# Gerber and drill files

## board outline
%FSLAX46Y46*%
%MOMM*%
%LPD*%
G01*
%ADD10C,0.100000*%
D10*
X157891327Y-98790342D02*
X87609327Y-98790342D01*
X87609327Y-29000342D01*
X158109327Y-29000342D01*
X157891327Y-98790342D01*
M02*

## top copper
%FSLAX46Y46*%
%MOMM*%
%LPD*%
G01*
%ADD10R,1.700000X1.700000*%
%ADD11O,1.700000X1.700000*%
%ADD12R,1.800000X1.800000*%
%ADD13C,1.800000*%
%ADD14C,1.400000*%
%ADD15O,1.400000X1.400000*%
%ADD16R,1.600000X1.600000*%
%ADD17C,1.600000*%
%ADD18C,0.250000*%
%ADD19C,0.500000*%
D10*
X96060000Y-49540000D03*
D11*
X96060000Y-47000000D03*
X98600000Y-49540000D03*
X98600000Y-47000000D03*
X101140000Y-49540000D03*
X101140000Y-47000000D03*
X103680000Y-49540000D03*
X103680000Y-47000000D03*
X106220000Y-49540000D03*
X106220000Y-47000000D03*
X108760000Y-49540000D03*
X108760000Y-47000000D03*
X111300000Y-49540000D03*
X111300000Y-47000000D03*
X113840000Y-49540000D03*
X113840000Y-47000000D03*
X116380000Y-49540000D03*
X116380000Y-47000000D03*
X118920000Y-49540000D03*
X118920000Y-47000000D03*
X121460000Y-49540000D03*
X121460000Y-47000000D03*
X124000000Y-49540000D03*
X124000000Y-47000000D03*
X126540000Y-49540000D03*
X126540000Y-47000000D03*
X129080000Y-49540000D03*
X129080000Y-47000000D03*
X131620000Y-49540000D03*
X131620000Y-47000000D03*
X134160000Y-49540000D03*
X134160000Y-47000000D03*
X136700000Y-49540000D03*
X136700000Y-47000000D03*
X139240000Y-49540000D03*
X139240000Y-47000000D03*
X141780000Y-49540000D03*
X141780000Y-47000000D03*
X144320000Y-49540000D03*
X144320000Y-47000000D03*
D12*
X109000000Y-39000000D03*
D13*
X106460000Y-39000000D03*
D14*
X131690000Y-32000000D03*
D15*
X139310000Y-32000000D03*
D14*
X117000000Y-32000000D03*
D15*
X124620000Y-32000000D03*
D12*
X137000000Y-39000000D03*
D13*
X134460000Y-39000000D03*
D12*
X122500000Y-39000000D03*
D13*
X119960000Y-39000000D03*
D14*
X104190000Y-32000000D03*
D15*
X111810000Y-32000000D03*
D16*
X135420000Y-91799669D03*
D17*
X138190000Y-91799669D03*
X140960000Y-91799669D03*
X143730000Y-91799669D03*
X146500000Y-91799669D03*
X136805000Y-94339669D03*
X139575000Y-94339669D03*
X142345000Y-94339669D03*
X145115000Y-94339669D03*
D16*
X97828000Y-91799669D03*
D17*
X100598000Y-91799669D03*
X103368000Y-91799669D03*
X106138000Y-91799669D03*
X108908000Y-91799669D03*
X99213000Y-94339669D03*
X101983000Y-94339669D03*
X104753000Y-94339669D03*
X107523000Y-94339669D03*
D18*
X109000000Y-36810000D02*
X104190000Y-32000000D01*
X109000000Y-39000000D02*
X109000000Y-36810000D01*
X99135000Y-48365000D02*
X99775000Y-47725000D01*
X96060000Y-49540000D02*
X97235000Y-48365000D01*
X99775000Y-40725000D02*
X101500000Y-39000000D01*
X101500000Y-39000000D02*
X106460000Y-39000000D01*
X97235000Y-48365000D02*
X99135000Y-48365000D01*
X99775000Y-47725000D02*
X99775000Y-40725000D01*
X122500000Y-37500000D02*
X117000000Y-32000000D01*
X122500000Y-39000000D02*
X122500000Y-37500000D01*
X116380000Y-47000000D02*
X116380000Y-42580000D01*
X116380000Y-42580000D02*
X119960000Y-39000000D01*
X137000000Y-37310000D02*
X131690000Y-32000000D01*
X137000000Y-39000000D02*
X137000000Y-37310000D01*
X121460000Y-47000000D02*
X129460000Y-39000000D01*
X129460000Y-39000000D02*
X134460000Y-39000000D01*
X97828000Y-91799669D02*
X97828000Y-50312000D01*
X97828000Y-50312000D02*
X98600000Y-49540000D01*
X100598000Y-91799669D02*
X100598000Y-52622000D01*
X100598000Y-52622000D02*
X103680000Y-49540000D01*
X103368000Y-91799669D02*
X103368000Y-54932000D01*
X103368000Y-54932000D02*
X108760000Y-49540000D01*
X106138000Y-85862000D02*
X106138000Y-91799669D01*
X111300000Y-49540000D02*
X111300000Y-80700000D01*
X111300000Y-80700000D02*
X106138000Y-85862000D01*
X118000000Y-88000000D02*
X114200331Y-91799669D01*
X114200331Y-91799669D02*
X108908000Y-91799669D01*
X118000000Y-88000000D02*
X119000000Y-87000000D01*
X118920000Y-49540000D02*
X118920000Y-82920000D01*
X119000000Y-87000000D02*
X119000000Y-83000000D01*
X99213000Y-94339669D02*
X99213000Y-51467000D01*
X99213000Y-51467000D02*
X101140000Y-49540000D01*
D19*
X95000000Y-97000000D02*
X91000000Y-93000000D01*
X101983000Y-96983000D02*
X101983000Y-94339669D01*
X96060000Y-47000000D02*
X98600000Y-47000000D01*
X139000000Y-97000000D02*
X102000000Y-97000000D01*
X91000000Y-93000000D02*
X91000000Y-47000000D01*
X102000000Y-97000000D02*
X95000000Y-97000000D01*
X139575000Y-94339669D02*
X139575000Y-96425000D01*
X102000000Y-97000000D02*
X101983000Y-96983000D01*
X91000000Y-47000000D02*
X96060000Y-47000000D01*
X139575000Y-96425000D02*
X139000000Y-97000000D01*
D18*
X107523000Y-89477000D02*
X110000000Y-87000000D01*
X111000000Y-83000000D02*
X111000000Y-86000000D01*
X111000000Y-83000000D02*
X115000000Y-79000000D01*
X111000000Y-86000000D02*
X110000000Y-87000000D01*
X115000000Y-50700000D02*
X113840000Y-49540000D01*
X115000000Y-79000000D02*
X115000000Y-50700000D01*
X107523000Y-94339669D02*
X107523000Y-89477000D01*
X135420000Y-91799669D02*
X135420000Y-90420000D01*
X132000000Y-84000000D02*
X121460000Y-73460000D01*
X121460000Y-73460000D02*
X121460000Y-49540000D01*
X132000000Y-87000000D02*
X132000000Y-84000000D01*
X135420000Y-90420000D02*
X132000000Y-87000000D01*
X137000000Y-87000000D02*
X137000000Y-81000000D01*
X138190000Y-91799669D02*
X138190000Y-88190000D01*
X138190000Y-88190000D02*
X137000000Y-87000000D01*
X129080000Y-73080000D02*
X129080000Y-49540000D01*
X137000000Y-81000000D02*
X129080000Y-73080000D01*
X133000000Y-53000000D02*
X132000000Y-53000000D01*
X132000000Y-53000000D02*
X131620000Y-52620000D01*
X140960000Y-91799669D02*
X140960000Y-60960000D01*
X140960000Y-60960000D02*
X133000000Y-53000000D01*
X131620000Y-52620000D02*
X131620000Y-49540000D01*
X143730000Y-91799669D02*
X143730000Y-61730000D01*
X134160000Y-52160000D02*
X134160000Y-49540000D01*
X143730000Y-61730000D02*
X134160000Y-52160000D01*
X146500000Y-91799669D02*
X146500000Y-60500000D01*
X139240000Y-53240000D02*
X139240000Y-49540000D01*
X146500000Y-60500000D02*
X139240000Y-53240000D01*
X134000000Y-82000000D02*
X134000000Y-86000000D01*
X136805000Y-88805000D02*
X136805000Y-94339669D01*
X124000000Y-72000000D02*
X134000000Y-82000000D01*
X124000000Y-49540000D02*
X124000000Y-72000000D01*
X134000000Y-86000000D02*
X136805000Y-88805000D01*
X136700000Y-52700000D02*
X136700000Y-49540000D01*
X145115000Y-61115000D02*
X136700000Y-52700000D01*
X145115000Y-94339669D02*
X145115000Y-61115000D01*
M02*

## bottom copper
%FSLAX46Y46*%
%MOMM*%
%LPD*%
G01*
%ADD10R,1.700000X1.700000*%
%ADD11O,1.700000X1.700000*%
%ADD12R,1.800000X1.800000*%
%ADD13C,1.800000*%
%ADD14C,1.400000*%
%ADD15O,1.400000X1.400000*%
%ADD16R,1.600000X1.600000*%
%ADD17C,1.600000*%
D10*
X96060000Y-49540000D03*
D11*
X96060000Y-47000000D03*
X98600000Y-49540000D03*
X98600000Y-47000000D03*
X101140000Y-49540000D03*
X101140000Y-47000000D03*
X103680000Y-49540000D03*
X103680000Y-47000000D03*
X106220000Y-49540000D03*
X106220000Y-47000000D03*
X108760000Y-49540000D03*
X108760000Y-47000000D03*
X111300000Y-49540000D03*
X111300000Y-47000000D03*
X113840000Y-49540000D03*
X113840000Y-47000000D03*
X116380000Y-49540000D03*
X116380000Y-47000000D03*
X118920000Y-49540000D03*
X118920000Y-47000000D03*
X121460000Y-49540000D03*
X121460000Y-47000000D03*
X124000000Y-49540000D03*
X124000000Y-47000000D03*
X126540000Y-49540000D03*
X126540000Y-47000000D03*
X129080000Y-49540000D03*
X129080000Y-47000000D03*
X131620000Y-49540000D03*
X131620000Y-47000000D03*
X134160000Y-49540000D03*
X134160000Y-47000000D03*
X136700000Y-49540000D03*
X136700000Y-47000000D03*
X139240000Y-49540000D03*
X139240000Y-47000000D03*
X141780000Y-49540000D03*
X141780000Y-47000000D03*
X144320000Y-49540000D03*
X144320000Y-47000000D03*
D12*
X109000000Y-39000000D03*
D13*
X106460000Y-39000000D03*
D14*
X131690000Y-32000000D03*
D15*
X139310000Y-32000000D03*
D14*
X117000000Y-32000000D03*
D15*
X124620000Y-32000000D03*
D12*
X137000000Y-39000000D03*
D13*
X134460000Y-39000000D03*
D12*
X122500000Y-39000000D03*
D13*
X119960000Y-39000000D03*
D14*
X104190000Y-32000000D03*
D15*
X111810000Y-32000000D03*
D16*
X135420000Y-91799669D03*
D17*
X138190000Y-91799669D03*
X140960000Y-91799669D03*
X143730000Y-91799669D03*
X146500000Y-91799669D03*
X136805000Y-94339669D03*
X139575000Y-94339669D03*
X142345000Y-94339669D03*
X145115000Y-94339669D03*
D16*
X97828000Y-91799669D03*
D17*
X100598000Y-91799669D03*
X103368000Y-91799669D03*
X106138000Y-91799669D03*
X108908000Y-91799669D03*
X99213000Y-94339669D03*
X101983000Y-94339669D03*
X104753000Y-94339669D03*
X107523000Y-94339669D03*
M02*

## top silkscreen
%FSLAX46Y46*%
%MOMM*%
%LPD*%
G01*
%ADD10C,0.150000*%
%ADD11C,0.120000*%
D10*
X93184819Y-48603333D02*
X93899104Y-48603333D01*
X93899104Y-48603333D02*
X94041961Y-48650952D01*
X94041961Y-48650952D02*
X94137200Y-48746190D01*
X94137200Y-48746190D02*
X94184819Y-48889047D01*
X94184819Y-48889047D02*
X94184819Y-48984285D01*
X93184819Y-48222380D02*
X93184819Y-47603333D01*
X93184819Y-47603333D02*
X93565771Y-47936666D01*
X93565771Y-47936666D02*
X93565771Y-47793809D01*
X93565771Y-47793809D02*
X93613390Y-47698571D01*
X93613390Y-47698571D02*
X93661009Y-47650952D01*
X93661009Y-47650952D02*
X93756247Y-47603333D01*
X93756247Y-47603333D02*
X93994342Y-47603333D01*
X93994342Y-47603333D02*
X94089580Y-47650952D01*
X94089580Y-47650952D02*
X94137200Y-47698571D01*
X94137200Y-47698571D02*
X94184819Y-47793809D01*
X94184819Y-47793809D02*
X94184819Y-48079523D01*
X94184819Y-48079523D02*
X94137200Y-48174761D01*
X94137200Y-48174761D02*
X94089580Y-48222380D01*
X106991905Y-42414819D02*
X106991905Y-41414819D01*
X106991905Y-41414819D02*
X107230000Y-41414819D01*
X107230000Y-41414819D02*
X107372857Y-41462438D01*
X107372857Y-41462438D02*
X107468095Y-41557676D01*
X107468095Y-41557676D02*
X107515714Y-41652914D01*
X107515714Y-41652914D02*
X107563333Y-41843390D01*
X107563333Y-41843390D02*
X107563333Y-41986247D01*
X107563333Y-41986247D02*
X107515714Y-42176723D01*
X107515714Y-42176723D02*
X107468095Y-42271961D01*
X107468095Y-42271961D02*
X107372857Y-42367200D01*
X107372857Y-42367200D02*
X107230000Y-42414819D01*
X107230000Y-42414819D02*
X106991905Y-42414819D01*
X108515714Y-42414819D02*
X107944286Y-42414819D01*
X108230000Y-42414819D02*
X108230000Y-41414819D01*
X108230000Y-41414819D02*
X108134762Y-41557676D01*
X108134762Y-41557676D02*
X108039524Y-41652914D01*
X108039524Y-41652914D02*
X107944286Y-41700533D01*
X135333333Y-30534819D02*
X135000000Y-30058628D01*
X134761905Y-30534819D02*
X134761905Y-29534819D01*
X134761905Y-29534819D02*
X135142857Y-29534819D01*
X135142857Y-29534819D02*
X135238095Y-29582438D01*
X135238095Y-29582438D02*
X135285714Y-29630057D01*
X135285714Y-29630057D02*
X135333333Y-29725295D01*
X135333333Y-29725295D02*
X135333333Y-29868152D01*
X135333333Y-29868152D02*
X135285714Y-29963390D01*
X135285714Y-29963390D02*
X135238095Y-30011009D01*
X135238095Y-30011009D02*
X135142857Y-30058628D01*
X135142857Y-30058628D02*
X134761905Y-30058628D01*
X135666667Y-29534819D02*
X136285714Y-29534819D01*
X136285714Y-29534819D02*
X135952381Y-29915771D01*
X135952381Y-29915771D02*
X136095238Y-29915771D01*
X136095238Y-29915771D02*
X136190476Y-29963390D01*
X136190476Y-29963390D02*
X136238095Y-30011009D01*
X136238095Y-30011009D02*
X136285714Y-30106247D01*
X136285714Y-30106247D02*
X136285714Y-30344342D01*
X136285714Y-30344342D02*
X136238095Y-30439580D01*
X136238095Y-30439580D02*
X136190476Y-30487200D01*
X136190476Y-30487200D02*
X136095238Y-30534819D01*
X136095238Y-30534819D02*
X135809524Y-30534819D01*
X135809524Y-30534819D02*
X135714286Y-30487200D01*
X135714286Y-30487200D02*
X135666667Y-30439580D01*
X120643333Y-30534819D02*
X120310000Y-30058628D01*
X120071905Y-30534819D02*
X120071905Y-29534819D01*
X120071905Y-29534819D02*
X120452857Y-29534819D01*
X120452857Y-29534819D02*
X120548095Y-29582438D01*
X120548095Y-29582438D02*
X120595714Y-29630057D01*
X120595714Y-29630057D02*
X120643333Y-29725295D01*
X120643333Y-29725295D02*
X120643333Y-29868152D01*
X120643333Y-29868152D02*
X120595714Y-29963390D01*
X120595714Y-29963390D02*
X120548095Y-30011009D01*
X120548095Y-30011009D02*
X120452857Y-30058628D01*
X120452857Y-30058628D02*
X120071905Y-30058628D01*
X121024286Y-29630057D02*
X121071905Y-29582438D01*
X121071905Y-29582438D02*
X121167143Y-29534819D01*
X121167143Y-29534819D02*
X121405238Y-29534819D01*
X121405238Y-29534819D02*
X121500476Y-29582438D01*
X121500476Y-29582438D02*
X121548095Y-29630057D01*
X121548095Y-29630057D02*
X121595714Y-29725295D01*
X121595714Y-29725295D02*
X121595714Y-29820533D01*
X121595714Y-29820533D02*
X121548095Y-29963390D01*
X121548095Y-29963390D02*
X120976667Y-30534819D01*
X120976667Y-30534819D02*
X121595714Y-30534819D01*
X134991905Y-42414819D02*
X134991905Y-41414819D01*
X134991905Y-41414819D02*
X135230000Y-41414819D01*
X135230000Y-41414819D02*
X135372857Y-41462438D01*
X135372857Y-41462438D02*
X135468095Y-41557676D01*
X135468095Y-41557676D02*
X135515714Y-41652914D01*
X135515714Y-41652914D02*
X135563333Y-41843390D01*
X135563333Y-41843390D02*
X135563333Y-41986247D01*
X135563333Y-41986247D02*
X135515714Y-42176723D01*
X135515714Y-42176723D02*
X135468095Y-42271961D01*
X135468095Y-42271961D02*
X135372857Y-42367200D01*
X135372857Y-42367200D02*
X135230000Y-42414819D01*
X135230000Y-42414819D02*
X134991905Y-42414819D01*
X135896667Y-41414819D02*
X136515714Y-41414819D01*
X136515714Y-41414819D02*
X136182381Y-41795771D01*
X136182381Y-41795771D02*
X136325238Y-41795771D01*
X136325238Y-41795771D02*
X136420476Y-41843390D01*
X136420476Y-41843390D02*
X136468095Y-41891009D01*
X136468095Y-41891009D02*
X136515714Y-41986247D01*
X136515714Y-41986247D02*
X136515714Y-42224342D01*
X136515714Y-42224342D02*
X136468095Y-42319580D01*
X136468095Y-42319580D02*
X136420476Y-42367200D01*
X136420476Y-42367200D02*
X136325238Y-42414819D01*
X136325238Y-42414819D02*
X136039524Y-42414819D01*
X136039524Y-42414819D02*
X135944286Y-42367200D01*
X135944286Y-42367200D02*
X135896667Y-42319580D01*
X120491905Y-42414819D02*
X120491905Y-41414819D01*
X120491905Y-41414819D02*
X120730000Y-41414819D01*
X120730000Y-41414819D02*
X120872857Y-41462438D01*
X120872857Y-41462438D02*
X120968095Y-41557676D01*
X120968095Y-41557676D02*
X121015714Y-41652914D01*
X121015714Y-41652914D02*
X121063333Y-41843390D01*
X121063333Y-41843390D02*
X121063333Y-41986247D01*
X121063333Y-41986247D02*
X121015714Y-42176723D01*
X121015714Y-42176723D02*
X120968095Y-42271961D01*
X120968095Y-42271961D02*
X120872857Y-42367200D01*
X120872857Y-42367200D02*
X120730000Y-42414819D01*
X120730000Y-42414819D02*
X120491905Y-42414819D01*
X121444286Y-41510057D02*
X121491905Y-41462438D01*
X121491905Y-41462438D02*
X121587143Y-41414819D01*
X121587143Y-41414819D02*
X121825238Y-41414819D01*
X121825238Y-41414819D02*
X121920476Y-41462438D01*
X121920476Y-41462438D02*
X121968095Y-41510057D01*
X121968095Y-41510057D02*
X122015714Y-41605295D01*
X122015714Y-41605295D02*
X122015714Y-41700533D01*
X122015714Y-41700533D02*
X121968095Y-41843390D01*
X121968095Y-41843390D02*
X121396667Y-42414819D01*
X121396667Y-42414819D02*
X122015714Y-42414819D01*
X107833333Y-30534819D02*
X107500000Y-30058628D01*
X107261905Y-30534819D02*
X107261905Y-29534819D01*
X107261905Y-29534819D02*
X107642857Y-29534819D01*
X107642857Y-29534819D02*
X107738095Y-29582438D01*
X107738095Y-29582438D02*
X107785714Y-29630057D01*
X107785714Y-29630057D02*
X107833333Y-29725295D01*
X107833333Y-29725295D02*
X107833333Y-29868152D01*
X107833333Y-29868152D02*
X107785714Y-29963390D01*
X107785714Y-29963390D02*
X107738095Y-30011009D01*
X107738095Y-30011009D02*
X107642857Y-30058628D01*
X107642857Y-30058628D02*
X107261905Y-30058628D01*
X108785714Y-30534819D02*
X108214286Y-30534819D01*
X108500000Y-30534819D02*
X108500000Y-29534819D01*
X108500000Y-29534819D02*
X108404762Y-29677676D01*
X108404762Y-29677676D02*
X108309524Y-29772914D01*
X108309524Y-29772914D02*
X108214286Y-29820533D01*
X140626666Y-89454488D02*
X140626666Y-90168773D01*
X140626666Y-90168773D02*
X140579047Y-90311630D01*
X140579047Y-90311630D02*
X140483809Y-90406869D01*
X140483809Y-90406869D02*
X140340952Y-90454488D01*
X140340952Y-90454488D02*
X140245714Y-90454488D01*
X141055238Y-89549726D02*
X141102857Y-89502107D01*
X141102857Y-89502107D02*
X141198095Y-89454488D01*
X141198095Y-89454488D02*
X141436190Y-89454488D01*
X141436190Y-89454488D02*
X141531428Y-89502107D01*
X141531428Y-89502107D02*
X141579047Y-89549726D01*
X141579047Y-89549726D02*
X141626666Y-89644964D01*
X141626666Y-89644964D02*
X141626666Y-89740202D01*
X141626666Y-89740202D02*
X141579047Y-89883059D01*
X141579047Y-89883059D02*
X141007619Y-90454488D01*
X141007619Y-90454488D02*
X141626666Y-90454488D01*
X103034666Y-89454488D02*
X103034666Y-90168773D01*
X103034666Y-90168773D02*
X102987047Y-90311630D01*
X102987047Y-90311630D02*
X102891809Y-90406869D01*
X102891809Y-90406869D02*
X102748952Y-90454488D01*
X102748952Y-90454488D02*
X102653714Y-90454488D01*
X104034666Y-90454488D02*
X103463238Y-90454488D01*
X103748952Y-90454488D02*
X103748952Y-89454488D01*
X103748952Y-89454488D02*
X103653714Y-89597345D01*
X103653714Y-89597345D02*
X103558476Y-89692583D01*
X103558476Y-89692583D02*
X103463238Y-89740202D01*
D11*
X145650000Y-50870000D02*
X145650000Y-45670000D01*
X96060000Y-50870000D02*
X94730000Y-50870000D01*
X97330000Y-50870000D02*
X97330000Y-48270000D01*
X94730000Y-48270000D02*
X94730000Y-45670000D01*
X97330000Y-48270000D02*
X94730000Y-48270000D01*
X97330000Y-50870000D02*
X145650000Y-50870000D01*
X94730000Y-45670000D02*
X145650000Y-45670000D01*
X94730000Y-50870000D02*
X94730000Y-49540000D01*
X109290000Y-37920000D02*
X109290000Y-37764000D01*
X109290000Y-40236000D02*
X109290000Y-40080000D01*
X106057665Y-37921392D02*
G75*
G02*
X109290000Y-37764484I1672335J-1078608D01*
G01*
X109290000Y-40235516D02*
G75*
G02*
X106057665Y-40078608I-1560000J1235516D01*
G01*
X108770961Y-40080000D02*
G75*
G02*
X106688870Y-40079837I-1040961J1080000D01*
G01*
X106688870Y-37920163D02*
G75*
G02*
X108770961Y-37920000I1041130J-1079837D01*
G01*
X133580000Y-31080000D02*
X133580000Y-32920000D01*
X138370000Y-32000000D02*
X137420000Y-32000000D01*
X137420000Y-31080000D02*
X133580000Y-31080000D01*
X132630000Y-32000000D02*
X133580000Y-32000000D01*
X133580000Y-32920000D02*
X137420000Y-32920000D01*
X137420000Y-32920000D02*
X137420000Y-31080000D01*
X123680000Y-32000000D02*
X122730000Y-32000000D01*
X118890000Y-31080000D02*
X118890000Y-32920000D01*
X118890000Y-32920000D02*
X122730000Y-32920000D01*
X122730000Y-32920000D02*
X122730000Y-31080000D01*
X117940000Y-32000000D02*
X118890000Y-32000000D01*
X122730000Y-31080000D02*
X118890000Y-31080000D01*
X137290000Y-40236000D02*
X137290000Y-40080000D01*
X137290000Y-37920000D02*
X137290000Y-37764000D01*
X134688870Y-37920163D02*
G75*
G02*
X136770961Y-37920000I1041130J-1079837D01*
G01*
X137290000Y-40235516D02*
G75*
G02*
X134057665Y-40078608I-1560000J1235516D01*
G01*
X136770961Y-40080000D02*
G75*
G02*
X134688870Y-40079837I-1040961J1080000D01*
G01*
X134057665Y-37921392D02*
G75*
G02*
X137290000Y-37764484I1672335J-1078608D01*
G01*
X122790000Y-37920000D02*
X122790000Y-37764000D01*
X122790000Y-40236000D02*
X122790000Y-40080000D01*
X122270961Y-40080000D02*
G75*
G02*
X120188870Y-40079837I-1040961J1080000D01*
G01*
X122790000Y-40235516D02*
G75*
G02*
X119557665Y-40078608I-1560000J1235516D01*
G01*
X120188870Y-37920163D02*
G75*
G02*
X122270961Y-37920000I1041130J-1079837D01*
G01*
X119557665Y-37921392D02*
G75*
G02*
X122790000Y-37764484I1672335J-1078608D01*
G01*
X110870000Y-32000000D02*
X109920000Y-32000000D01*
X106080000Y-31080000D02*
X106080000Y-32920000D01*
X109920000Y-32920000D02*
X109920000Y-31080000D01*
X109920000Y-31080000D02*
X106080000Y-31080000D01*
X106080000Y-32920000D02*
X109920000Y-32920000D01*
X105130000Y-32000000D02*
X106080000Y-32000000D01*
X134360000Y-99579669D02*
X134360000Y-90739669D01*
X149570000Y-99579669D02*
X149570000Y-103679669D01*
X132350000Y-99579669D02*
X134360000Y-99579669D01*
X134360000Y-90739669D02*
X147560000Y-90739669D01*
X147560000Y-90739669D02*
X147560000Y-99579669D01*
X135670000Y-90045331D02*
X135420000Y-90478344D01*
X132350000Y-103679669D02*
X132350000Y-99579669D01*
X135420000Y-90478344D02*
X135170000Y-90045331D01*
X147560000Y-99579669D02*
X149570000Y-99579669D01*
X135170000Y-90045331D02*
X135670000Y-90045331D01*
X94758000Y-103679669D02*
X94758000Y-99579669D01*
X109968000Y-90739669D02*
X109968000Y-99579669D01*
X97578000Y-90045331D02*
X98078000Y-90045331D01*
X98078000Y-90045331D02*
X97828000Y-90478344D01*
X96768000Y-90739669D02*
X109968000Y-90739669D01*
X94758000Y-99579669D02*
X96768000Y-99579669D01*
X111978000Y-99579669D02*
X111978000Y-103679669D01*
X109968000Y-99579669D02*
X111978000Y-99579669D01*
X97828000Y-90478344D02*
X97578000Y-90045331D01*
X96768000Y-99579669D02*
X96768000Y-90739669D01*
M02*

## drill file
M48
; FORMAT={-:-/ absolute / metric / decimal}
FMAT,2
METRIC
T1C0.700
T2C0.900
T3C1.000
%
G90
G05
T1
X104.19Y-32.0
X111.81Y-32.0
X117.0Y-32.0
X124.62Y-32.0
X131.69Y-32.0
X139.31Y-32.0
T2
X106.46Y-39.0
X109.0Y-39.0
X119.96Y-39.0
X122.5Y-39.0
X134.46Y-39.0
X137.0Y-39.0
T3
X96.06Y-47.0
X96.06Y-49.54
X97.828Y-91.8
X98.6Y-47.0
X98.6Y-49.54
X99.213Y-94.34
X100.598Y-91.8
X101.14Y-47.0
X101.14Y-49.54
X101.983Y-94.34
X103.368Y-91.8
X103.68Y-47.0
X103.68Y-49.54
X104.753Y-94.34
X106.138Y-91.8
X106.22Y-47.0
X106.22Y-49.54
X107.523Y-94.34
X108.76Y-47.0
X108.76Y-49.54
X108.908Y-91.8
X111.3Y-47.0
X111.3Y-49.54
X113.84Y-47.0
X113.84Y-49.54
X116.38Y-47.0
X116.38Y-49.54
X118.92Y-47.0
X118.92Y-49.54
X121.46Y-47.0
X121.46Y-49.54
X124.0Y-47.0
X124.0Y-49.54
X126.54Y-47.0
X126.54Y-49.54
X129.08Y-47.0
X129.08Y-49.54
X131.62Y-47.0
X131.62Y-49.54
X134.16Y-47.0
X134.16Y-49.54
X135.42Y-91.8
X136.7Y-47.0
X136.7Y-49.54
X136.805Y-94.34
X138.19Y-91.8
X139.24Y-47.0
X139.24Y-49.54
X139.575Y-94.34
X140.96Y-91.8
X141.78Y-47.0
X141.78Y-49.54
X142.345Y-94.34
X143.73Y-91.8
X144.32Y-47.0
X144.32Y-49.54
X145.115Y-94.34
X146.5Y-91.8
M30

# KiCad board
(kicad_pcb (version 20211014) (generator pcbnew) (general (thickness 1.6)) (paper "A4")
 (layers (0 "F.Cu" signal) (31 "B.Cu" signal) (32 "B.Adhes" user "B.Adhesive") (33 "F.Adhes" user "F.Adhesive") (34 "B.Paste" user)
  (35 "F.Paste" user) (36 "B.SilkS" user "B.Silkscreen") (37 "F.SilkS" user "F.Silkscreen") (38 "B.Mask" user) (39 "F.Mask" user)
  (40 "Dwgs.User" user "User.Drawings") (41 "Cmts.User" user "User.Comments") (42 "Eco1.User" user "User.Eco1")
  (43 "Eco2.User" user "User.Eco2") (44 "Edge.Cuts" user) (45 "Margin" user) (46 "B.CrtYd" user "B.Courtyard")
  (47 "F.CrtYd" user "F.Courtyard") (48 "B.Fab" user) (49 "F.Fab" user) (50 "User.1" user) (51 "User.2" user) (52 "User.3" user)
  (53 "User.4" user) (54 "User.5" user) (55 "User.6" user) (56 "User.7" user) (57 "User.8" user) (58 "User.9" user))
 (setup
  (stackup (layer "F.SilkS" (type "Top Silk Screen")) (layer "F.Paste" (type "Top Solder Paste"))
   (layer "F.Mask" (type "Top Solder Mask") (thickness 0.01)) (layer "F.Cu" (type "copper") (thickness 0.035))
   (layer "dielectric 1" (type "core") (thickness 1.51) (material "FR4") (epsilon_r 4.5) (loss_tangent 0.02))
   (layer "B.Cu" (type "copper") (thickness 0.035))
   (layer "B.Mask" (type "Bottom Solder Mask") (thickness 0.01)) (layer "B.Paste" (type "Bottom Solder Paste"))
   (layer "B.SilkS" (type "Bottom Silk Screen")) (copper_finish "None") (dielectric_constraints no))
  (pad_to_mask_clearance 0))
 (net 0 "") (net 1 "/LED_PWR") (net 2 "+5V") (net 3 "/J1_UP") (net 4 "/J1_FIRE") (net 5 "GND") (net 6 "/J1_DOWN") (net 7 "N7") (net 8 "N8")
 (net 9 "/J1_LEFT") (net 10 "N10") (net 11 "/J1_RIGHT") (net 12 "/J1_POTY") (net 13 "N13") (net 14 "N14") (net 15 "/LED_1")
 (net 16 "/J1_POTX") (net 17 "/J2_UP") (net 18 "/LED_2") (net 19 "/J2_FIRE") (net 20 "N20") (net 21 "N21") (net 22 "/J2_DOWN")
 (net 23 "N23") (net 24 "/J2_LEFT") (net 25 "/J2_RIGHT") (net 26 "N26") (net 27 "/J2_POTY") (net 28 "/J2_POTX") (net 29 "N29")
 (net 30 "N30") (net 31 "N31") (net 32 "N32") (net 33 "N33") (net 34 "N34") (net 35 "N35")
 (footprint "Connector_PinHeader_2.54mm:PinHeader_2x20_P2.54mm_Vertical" (layer "F.Cu") (at 96.06 49.54 90)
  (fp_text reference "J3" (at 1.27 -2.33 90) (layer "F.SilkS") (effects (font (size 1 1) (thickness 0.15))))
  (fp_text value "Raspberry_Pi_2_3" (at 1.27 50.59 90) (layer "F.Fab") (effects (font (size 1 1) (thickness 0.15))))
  (fp_line (start -1.33 49.59) (end 3.87 49.59) (layer "F.SilkS") (width 0.12))
  (fp_line (start -1.33 0) (end -1.33 -1.33) (layer "F.SilkS") (width 0.12))
  (fp_line (start -1.33 1.27) (end 1.27 1.27) (layer "F.SilkS") (width 0.12))
  (fp_line (start 1.27 -1.33) (end 3.87 -1.33) (layer "F.SilkS") (width 0.12))
  (fp_line (start 1.27 1.27) (end 1.27 -1.33) (layer "F.SilkS") (width 0.12))
  (fp_line (start -1.33 1.27) (end -1.33 49.59) (layer "F.SilkS") (width 0.12))
  (fp_line (start 3.87 -1.33) (end 3.87 49.59) (layer "F.SilkS") (width 0.12))
  (fp_line (start -1.33 -1.33) (end 0 -1.33) (layer "F.SilkS") (width 0.12))
  (pad "1" thru_hole rect (at 0 0 90) (size 1.7 1.7) (drill 1) (layers *.Cu *.Mask) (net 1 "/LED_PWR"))
  (pad "2" thru_hole oval (at 2.54 0 90) (size 1.7 1.7) (drill 1) (layers *.Cu *.Mask) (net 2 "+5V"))
  (pad "3" thru_hole oval (at 0 2.54 90) (size 1.7 1.7) (drill 1) (layers *.Cu *.Mask) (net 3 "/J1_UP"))
  (pad "4" thru_hole oval (at 2.54 2.54 90) (size 1.7 1.7) (drill 1) (layers *.Cu *.Mask) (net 2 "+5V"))
  (pad "5" thru_hole oval (at 0 5.08 90) (size 1.7 1.7) (drill 1) (layers *.Cu *.Mask) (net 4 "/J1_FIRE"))
  (pad "6" thru_hole oval (at 2.54 5.08 90) (size 1.7 1.7) (drill 1) (layers *.Cu *.Mask) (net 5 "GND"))
  (pad "7" thru_hole oval (at 0 7.62 90) (size 1.7 1.7) (drill 1) (layers *.Cu *.Mask) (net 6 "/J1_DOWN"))
  (pad "8" thru_hole oval (at 2.54 7.62 90) (size 1.7 1.7) (drill 1) (layers *.Cu *.Mask) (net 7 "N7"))
  (pad "9" thru_hole oval (at 0 10.16 90) (size 1.7 1.7) (drill 1) (layers *.Cu *.Mask) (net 5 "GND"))
  (pad "10" thru_hole oval (at 2.54 10.16 90) (size 1.7 1.7) (drill 1) (layers *.Cu *.Mask) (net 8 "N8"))
  (pad "11" thru_hole oval (at 0 12.7 90) (size 1.7 1.7) (drill 1) (layers *.Cu *.Mask) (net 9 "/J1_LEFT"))
  (pad "12" thru_hole oval (at 2.54 12.7 90) (size 1.7 1.7) (drill 1) (layers *.Cu *.Mask) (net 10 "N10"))
  (pad "13" thru_hole oval (at 0 15.24 90) (size 1.7 1.7) (drill 1) (layers *.Cu *.Mask) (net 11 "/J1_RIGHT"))
  (pad "14" thru_hole oval (at 2.54 15.24 90) (size 1.7 1.7) (drill 1) (layers *.Cu *.Mask) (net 5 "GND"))
  (pad "15" thru_hole oval (at 0 17.78 90) (size 1.7 1.7) (drill 1) (layers *.Cu *.Mask) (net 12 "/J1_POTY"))
  (pad "16" thru_hole oval (at 2.54 17.78 90) (size 1.7 1.7) (drill 1) (layers *.Cu *.Mask) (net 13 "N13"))
  (pad "17" thru_hole oval (at 0 20.32 90) (size 1.7 1.7) (drill 1) (layers *.Cu *.Mask) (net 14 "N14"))
  (pad "18" thru_hole oval (at 2.54 20.32 90) (size 1.7 1.7) (drill 1) (layers *.Cu *.Mask) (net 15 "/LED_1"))
  (pad "19" thru_hole oval (at 0 22.86 90) (size 1.7 1.7) (drill 1) (layers *.Cu *.Mask) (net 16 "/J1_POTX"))
  (pad "20" thru_hole oval (at 2.54 22.86 90) (size 1.7 1.7) (drill 1) (layers *.Cu *.Mask) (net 5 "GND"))
  (pad "21" thru_hole oval (at 0 25.4 90) (size 1.7 1.7) (drill 1) (layers *.Cu *.Mask) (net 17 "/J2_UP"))
  (pad "22" thru_hole oval (at 2.54 25.4 90) (size 1.7 1.7) (drill 1) (layers *.Cu *.Mask) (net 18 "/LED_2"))
  (pad "23" thru_hole oval (at 0 27.94 90) (size 1.7 1.7) (drill 1) (layers *.Cu *.Mask) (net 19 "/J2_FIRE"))
  (pad "24" thru_hole oval (at 2.54 27.94 90) (size 1.7 1.7) (drill 1) (layers *.Cu *.Mask) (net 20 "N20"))
  (pad "25" thru_hole oval (at 0 30.48 90) (size 1.7 1.7) (drill 1) (layers *.Cu *.Mask) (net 5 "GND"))
  (pad "26" thru_hole oval (at 2.54 30.48 90) (size 1.7 1.7) (drill 1) (layers *.Cu *.Mask) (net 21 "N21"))
  (pad "27" thru_hole oval (at 0 33.02 90) (size 1.7 1.7) (drill 1) (layers *.Cu *.Mask) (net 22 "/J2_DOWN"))
  (pad "28" thru_hole oval (at 2.54 33.02 90) (size 1.7 1.7) (drill 1) (layers *.Cu *.Mask) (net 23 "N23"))
  (pad "29" thru_hole oval (at 0 35.56 90) (size 1.7 1.7) (drill 1) (layers *.Cu *.Mask) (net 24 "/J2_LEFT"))
  (pad "30" thru_hole oval (at 2.54 35.56 90) (size 1.7 1.7) (drill 1) (layers *.Cu *.Mask) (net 5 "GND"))
  (pad "31" thru_hole oval (at 0 38.1 90) (size 1.7 1.7) (drill 1) (layers *.Cu *.Mask) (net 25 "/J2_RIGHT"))
  (pad "32" thru_hole oval (at 2.54 38.1 90) (size 1.7 1.7) (drill 1) (layers *.Cu *.Mask) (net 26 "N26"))
  (pad "33" thru_hole oval (at 0 40.64 90) (size 1.7 1.7) (drill 1) (layers *.Cu *.Mask) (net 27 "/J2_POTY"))
  (pad "34" thru_hole oval (at 2.54 40.64 90) (size 1.7 1.7) (drill 1) (layers *.Cu *.Mask) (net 5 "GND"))
  (pad "35" thru_hole oval (at 0 43.18 90) (size 1.7 1.7) (drill 1) (layers *.Cu *.Mask) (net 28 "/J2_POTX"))
  (pad "36" thru_hole oval (at 2.54 43.18 90) (size 1.7 1.7) (drill 1) (layers *.Cu *.Mask) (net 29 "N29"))
  (pad "37" thru_hole oval (at 0 45.72 90) (size 1.7 1.7) (drill 1) (layers *.Cu *.Mask) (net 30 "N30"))
  (pad "38" thru_hole oval (at 2.54 45.72 90) (size 1.7 1.7) (drill 1) (layers *.Cu *.Mask) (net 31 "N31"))
  (pad "39" thru_hole oval (at 0 48.26 90) (size 1.7 1.7) (drill 1) (layers *.Cu *.Mask) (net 5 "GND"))
  (pad "40" thru_hole oval (at 2.54 48.26 90) (size 1.7 1.7) (drill 1) (layers *.Cu *.Mask) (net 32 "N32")))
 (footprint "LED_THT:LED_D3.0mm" (layer "F.Cu") (at 109 39 180)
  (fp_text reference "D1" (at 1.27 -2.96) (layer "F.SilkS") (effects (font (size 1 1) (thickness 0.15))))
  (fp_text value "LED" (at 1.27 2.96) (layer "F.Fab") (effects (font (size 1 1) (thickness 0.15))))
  (fp_line (start -0.29 1.08) (end -0.29 1.236) (layer "F.SilkS") (width 0.12))
  (fp_line (start -0.29 -1.236) (end -0.29 -1.08) (layer "F.SilkS") (width 0.12))
  (fp_arc (start 2.942335 1.078608) (mid 1.366487 1.987659) (end -0.29 1.235516) (layer "F.SilkS") (width 0.12))
  (fp_arc (start -0.29 -1.235516) (mid 1.366487 -1.987659) (end 2.942335 -1.078608) (layer "F.SilkS") (width 0.12))
  (fp_arc (start 0.229039 -1.08) (mid 1.270117 -1.5) (end 2.31113 -1.079837) (layer "F.SilkS") (width 0.12))
  (fp_arc (start 2.31113 1.079837) (mid 1.270117 1.5) (end 0.229039 1.08) (layer "F.SilkS") (width 0.12))
  (pad "1" thru_hole rect (at 0 0 180) (size 1.8 1.8) (drill 0.9) (layers *.Cu *.Mask) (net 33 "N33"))
  (pad "2" thru_hole circle (at 2.54 0 180) (size 1.8 1.8) (drill 0.9) (layers *.Cu *.Mask) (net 1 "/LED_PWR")))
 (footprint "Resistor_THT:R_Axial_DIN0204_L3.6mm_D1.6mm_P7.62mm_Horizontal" (layer "F.Cu") (at 131.69 32)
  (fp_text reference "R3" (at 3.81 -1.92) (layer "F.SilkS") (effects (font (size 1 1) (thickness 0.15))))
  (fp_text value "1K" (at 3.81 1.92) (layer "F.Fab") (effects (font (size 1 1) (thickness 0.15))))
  (fp_line (start 1.89 -0.92) (end 1.89 0.92) (layer "F.SilkS") (width 0.12))
  (fp_line (start 6.68 0) (end 5.73 0) (layer "F.SilkS") (width 0.12))
  (fp_line (start 5.73 -0.92) (end 1.89 -0.92) (layer "F.SilkS") (width 0.12))
  (fp_line (start 0.94 0) (end 1.89 0) (layer "F.SilkS") (width 0.12))
  (fp_line (start 1.89 0.92) (end 5.73 0.92) (layer "F.SilkS") (width 0.12))
  (fp_line (start 5.73 0.92) (end 5.73 -0.92) (layer "F.SilkS") (width 0.12))
  (pad "1" thru_hole circle (at 0 0) (size 1.4 1.4) (drill 0.7) (layers *.Cu *.Mask) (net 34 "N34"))
  (pad "2" thru_hole oval (at 7.62 0) (size 1.4 1.4) (drill 0.7) (layers *.Cu *.Mask) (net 5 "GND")))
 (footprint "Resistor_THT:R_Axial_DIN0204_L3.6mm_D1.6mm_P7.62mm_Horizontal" (layer "F.Cu") (at 117 32)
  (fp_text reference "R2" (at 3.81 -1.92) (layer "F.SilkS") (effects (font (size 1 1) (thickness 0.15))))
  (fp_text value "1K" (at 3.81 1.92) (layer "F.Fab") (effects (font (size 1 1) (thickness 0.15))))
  (fp_line (start 6.68 0) (end 5.73 0) (layer "F.SilkS") (width 0.12))
  (fp_line (start 1.89 -0.92) (end 1.89 0.92) (layer "F.SilkS") (width 0.12))
  (fp_line (start 1.89 0.92) (end 5.73 0.92) (layer "F.SilkS") (width 0.12))
  (fp_line (start 5.73 0.92) (end 5.73 -0.92) (layer "F.SilkS") (width 0.12))
  (fp_line (start 0.94 0) (end 1.89 0) (layer "F.SilkS") (width 0.12))
  (fp_line (start 5.73 -0.92) (end 1.89 -0.92) (layer "F.SilkS") (width 0.12))
  (pad "1" thru_hole circle (at 0 0) (size 1.4 1.4) (drill 0.7) (layers *.Cu *.Mask) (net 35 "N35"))
  (pad "2" thru_hole oval (at 7.62 0) (size 1.4 1.4) (drill 0.7) (layers *.Cu *.Mask) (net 5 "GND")))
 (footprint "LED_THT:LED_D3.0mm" (layer "F.Cu") (at 137 39 180)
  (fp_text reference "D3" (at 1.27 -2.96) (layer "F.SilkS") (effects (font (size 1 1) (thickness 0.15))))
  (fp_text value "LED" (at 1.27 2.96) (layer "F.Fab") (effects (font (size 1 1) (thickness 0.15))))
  (fp_line (start -0.29 -1.236) (end -0.29 -1.08) (layer "F.SilkS") (width 0.12))
  (fp_line (start -0.29 1.08) (end -0.29 1.236) (layer "F.SilkS") (width 0.12))
  (fp_arc (start 2.31113 1.079837) (mid 1.270117 1.5) (end 0.229039 1.08) (layer "F.SilkS") (width 0.12))
  (fp_arc (start -0.29 -1.235516) (mid 1.366487 -1.987659) (end 2.942335 -1.078608) (layer "F.SilkS") (width 0.12))
  (fp_arc (start 0.229039 -1.08) (mid 1.270117 -1.5) (end 2.31113 -1.079837) (layer "F.SilkS") (width 0.12))
  (fp_arc (start 2.942335 1.078608) (mid 1.366487 1.987659) (end -0.29 1.235516) (layer "F.SilkS") (width 0.12))
  (pad "1" thru_hole rect (at 0 0 180) (size 1.8 1.8) (drill 0.9) (layers *.Cu *.Mask) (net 34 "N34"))
  (pad "2" thru_hole circle (at 2.54 0 180) (size 1.8 1.8) (drill 0.9) (layers *.Cu *.Mask) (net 18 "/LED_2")))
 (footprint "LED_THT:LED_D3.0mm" (layer "F.Cu") (at 122.5 39 180)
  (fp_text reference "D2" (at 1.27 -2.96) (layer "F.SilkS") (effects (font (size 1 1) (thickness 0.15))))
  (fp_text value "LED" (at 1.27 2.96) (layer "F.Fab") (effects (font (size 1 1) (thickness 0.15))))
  (fp_line (start -0.29 1.08) (end -0.29 1.236) (layer "F.SilkS") (width 0.12))
  (fp_line (start -0.29 -1.236) (end -0.29 -1.08) (layer "F.SilkS") (width 0.12))
  (fp_arc (start 0.229039 -1.08) (mid 1.270117 -1.5) (end 2.31113 -1.079837) (layer "F.SilkS") (width 0.12))
  (fp_arc (start -0.29 -1.235516) (mid 1.366487 -1.987659) (end 2.942335 -1.078608) (layer "F.SilkS") (width 0.12))
  (fp_arc (start 2.31113 1.079837) (mid 1.270117 1.5) (end 0.229039 1.08) (layer "F.SilkS") (width 0.12))
  (fp_arc (start 2.942335 1.078608) (mid 1.366487 1.987659) (end -0.29 1.235516) (layer "F.SilkS") (width 0.12))
  (pad "1" thru_hole rect (at 0 0 180) (size 1.8 1.8) (drill 0.9) (layers *.Cu *.Mask) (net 35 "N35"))
  (pad "2" thru_hole circle (at 2.54 0 180) (size 1.8 1.8) (drill 0.9) (layers *.Cu *.Mask) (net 15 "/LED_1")))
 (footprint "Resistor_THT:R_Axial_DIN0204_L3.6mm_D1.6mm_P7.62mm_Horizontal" (layer "F.Cu") (at 104.19 32)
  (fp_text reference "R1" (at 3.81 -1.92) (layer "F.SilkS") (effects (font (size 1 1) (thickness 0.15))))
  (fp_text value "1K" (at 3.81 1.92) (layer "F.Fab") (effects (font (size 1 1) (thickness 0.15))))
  (fp_line (start 6.68 0) (end 5.73 0) (layer "F.SilkS") (width 0.12))
  (fp_line (start 1.89 -0.92) (end 1.89 0.92) (layer "F.SilkS") (width 0.12))
  (fp_line (start 5.73 0.92) (end 5.73 -0.92) (layer "F.SilkS") (width 0.12))
  (fp_line (start 5.73 -0.92) (end 1.89 -0.92) (layer "F.SilkS") (width 0.12))
  (fp_line (start 1.89 0.92) (end 5.73 0.92) (layer "F.SilkS") (width 0.12))
  (fp_line (start 0.94 0) (end 1.89 0) (layer "F.SilkS") (width 0.12))
  (pad "1" thru_hole circle (at 0 0) (size 1.4 1.4) (drill 0.7) (layers *.Cu *.Mask) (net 33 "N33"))
  (pad "2" thru_hole oval (at 7.62 0) (size 1.4 1.4) (drill 0.7) (layers *.Cu *.Mask) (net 5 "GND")))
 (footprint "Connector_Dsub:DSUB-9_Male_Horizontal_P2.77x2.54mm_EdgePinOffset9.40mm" (layer "F.Cu") (at 135.42 91.799669)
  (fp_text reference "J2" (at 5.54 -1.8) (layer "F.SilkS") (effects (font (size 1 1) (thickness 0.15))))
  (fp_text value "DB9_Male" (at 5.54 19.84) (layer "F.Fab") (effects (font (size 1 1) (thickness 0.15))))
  (fp_line (start -1.06 7.78) (end -1.06 -1.06) (layer "F.SilkS") (width 0.12))
  (fp_line (start 14.15 7.78) (end 14.15 11.88) (layer "F.SilkS") (width 0.12))
  (fp_line (start -3.07 7.78) (end -1.06 7.78) (layer "F.SilkS") (width 0.12))
  (fp_line (start -1.06 -1.06) (end 12.14 -1.06) (layer "F.SilkS") (width 0.12))
  (fp_line (start 12.14 -1.06) (end 12.14 7.78) (layer "F.SilkS") (width 0.12))
  (fp_line (start 0.25 -1.754338) (end 0 -1.321325) (layer "F.SilkS") (width 0.12))
  (fp_line (start -3.07 11.88) (end -3.07 7.78) (layer "F.SilkS") (width 0.12))
  (fp_line (start 0 -1.321325) (end -0.25 -1.754338) (layer "F.SilkS") (width 0.12))
  (fp_line (start 12.14 7.78) (end 14.15 7.78) (layer "F.SilkS") (width 0.12))
  (fp_line (start -0.25 -1.754338) (end 0.25 -1.754338) (layer "F.SilkS") (width 0.12))
  (pad "1" thru_hole rect (at 0 0) (size 1.6 1.6) (drill 1) (layers *.Cu *.Mask) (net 17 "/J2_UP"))
  (pad "2" thru_hole circle (at 2.77 0) (size 1.6 1.6) (drill 1) (layers *.Cu *.Mask) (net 22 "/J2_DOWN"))
  (pad "3" thru_hole circle (at 5.54 0) (size 1.6 1.6) (drill 1) (layers *.Cu *.Mask) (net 24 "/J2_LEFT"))
  (pad "4" thru_hole circle (at 8.31 0) (size 1.6 1.6) (drill 1) (layers *.Cu *.Mask) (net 25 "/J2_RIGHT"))
  (pad "5" thru_hole circle (at 11.08 0) (size 1.6 1.6) (drill 1) (layers *.Cu *.Mask) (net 28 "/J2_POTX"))
  (pad "6" thru_hole circle (at 1.385 2.54) (size 1.6 1.6) (drill 1) (layers *.Cu *.Mask) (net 19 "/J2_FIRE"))
  (pad "7" thru_hole circle (at 4.155 2.54) (size 1.6 1.6) (drill 1) (layers *.Cu *.Mask) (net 2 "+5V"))
  (pad "8" thru_hole circle (at 6.925 2.54) (size 1.6 1.6) (drill 1) (layers *.Cu *.Mask) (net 5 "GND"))
  (pad "9" thru_hole circle (at 9.695 2.54) (size 1.6 1.6) (drill 1) (layers *.Cu *.Mask) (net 27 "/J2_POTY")))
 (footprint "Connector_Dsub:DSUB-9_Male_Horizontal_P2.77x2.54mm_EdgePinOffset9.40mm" (layer "F.Cu") (at 97.828 91.799669)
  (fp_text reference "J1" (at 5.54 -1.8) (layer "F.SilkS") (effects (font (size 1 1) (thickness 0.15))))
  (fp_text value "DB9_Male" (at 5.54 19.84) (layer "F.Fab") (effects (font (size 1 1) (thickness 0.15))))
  (fp_line (start -3.07 11.88) (end -3.07 7.78) (layer "F.SilkS") (width 0.12))
  (fp_line (start 12.14 -1.06) (end 12.14 7.78) (layer "F.SilkS") (width 0.12))
  (fp_line (start -0.25 -1.754338) (end 0.25 -1.754338) (layer "F.SilkS") (width 0.12))
  (fp_line (start 0.25 -1.754338) (end 0 -1.321325) (layer "F.SilkS") (width 0.12))
  (fp_line (start -1.06 -1.06) (end 12.14 -1.06) (layer "F.SilkS") (width 0.12))
  (fp_line (start -3.07 7.78) (end -1.06 7.78) (layer "F.SilkS") (width 0.12))
  (fp_line (start 14.15 7.78) (end 14.15 11.88) (layer "F.SilkS") (width 0.12))
  (fp_line (start 12.14 7.78) (end 14.15 7.78) (layer "F.SilkS") (width 0.12))
  (fp_line (start 0 -1.321325) (end -0.25 -1.754338) (layer "F.SilkS") (width 0.12))
  (fp_line (start -1.06 7.78) (end -1.06 -1.06) (layer "F.SilkS") (width 0.12))
  (pad "1" thru_hole rect (at 0 0) (size 1.6 1.6) (drill 1) (layers *.Cu *.Mask) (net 3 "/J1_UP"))
  (pad "2" thru_hole circle (at 2.77 0) (size 1.6 1.6) (drill 1) (layers *.Cu *.Mask) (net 6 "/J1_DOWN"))
  (pad "3" thru_hole circle (at 5.54 0) (size 1.6 1.6) (drill 1) (layers *.Cu *.Mask) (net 9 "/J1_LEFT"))
  (pad "4" thru_hole circle (at 8.31 0) (size 1.6 1.6) (drill 1) (layers *.Cu *.Mask) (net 11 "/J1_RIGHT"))
  (pad "5" thru_hole circle (at 11.08 0) (size 1.6 1.6) (drill 1) (layers *.Cu *.Mask) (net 16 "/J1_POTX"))
  (pad "6" thru_hole circle (at 1.385 2.54) (size 1.6 1.6) (drill 1) (layers *.Cu *.Mask) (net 4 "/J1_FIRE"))
  (pad "7" thru_hole circle (at 4.155 2.54) (size 1.6 1.6) (drill 1) (layers *.Cu *.Mask) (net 2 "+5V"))
  (pad "8" thru_hole circle (at 6.925 2.54) (size 1.6 1.6) (drill 1) (layers *.Cu *.Mask) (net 5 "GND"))
  (pad "9" thru_hole circle (at 9.695 2.54) (size 1.6 1.6) (drill 1) (layers *.Cu *.Mask) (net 12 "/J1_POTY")))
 (gr_poly
  (pts (xy 157.891327 98.790342) (xy 87.609327 98.790342) (xy 87.609327 29.000342) (xy 158.109327 29.000342)) (layer "Edge.Cuts")
  (width 0.1) (fill none))
 (segment (start 109 36.81) (end 104.19 32) (width 0.25) (layer "F.Cu") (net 33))
 (segment (start 109 39) (end 109 36.81) (width 0.25) (layer "F.Cu") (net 33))
 (segment (start 99.135 48.365) (end 99.775 47.725) (width 0.25) (layer "F.Cu") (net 1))
 (segment (start 96.06 49.54) (end 97.235 48.365) (width 0.25) (layer "F.Cu") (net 1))
 (segment (start 99.775 40.725) (end 101.5 39) (width 0.25) (layer "F.Cu") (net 1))
 (segment (start 101.5 39) (end 106.46 39) (width 0.25) (layer "F.Cu") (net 1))
 (segment (start 97.235 48.365) (end 99.135 48.365) (width 0.25) (layer "F.Cu") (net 1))
 (segment (start 99.775 47.725) (end 99.775 40.725) (width 0.25) (layer "F.Cu") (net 1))
 (segment (start 122.5 37.5) (end 117 32) (width 0.25) (layer "F.Cu") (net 35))
 (segment (start 122.5 39) (end 122.5 37.5) (width 0.25) (layer "F.Cu") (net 35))
 (segment (start 116.38 47) (end 116.38 42.58) (width 0.25) (layer "F.Cu") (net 15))
 (segment (start 116.38 42.58) (end 119.96 39) (width 0.25) (layer "F.Cu") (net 15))
 (segment (start 137 37.31) (end 131.69 32) (width 0.25) (layer "F.Cu") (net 34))
 (segment (start 137 39) (end 137 37.31) (width 0.25) (layer "F.Cu") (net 34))
 (segment (start 121.46 47) (end 129.46 39) (width 0.25) (layer "F.Cu") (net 18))
 (segment (start 129.46 39) (end 134.46 39) (width 0.25) (layer "F.Cu") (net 18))
 (segment (start 97.828 91.799669) (end 97.828 50.312) (width 0.25) (layer "F.Cu") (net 3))
 (segment (start 97.828 50.312) (end 98.6 49.54) (width 0.25) (layer "F.Cu") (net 3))
 (segment (start 100.598 91.799669) (end 100.598 52.622) (width 0.25) (layer "F.Cu") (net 6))
 (segment (start 100.598 52.622) (end 103.68 49.54) (width 0.25) (layer "F.Cu") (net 6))
 (segment (start 103.368 91.799669) (end 103.368 54.932) (width 0.25) (layer "F.Cu") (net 9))
 (segment (start 103.368 54.932) (end 108.76 49.54) (width 0.25) (layer "F.Cu") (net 9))
 (segment (start 106.138 85.862) (end 106.138 91.799669) (width 0.25) (layer "F.Cu") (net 11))
 (segment (start 111.3 49.54) (end 111.3 80.7) (width 0.25) (layer "F.Cu") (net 11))
 (segment (start 111.3 80.7) (end 106.138 85.862) (width 0.25) (layer "F.Cu") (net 11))
 (segment (start 118 88) (end 114.200331 91.799669) (width 0.25) (layer "F.Cu") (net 16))
 (segment (start 114.200331 91.799669) (end 108.908 91.799669) (width 0.25) (layer "F.Cu") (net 16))
 (segment (start 118 88) (end 119 87) (width 0.25) (layer "F.Cu") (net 16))
 (segment (start 118.92 49.54) (end 118.92 82.92) (width 0.25) (layer "F.Cu") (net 16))
 (segment (start 119 87) (end 119 83) (width 0.25) (layer "F.Cu") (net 16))
 (segment (start 99.213 94.339669) (end 99.213 51.467) (width 0.25) (layer "F.Cu") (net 4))
 (segment (start 99.213 51.467) (end 101.14 49.54) (width 0.25) (layer "F.Cu") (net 4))
 (segment (start 95 97) (end 91 93) (width 0.5) (layer "F.Cu") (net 2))
 (segment (start 101.983 96.983) (end 101.983 94.339669) (width 0.5) (layer "F.Cu") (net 2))
 (segment (start 96.06 47) (end 98.6 47) (width 0.5) (layer "F.Cu") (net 2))
 (segment (start 139 97) (end 102 97) (width 0.5) (layer "F.Cu") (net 2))
 (segment (start 91 93) (end 91 47) (width 0.5) (layer "F.Cu") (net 2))
 (segment (start 102 97) (end 95 97) (width 0.5) (layer "F.Cu") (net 2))
 (segment (start 139.575 94.339669) (end 139.575 96.425) (width 0.5) (layer "F.Cu") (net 2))
 (segment (start 102 97) (end 101.983 96.983) (width 0.5) (layer "F.Cu") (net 2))
 (segment (start 91 47) (end 96.06 47) (width 0.5) (layer "F.Cu") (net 2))
 (segment (start 139.575 96.425) (end 139 97) (width 0.5) (layer "F.Cu") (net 2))
 (segment (start 107.523 89.477) (end 110 87) (width 0.25) (layer "F.Cu") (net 12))
 (segment (start 111 83) (end 111 86) (width 0.25) (layer "F.Cu") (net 12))
 (segment (start 111 83) (end 115 79) (width 0.25) (layer "F.Cu") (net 12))
 (segment (start 111 86) (end 110 87) (width 0.25) (layer "F.Cu") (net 12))
 (segment (start 115 50.7) (end 113.84 49.54) (width 0.25) (layer "F.Cu") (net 12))
 (segment (start 115 79) (end 115 50.7) (width 0.25) (layer "F.Cu") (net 12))
 (segment (start 107.523 94.339669) (end 107.523 89.477) (width 0.25) (layer "F.Cu") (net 12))
 (segment (start 135.42 91.799669) (end 135.42 90.42) (width 0.25) (layer "F.Cu") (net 17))
 (segment (start 132 84) (end 121.46 73.46) (width 0.25) (layer "F.Cu") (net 17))
 (segment (start 121.46 73.46) (end 121.46 49.54) (width 0.25) (layer "F.Cu") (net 17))
 (segment (start 132 87) (end 132 84) (width 0.25) (layer "F.Cu") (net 17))
 (segment (start 135.42 90.42) (end 132 87) (width 0.25) (layer "F.Cu") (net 17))
 (segment (start 137 87) (end 137 81) (width 0.25) (layer "F.Cu") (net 22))
 (segment (start 138.19 91.799669) (end 138.19 88.19) (width 0.25) (layer "F.Cu") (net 22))
 (segment (start 138.19 88.19) (end 137 87) (width 0.25) (layer "F.Cu") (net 22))
 (segment (start 129.08 73.08) (end 129.08 49.54) (width 0.25) (layer "F.Cu") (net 22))
 (segment (start 137 81) (end 129.08 73.08) (width 0.25) (layer "F.Cu") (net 22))
 (segment (start 133 53) (end 132 53) (width 0.25) (layer "F.Cu") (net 24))
 (segment (start 132 53) (end 131.62 52.62) (width 0.25) (layer "F.Cu") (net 24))
 (segment (start 140.96 91.799669) (end 140.96 60.96) (width 0.25) (layer "F.Cu") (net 24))
 (segment (start 140.96 60.96) (end 133 53) (width 0.25) (layer "F.Cu") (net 24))
 (segment (start 131.62 52.62) (end 131.62 49.54) (width 0.25) (layer "F.Cu") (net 24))
 (segment (start 143.73 91.799669) (end 143.73 61.73) (width 0.25) (layer "F.Cu") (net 25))
 (segment (start 134.16 52.16) (end 134.16 49.54) (width 0.25) (layer "F.Cu") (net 25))
 (segment (start 143.73 61.73) (end 134.16 52.16) (width 0.25) (layer "F.Cu") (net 25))
 (segment (start 146.5 91.799669) (end 146.5 60.5) (width 0.25) (layer "F.Cu") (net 28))
 (segment (start 139.24 53.24) (end 139.24 49.54) (width 0.25) (layer "F.Cu") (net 28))
 (segment (start 146.5 60.5) (end 139.24 53.24) (width 0.25) (layer "F.Cu") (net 28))
 (segment (start 134 82) (end 134 86) (width 0.25) (layer "F.Cu") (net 19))
 (segment (start 136.805 88.805) (end 136.805 94.339669) (width 0.25) (layer "F.Cu") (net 19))
 (segment (start 124 72) (end 134 82) (width 0.25) (layer "F.Cu") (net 19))
 (segment (start 124 49.54) (end 124 72) (width 0.25) (layer "F.Cu") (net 19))
 (segment (start 134 86) (end 136.805 88.805) (width 0.25) (layer "F.Cu") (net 19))
 (segment (start 136.7 52.7) (end 136.7 49.54) (width 0.25) (layer "F.Cu") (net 27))
 (segment (start 145.115 61.115) (end 136.7 52.7) (width 0.25) (layer "F.Cu") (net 27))
 (segment (start 145.115 94.339669) (end 145.115 61.115) (width 0.25) (layer "F.Cu") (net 27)))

